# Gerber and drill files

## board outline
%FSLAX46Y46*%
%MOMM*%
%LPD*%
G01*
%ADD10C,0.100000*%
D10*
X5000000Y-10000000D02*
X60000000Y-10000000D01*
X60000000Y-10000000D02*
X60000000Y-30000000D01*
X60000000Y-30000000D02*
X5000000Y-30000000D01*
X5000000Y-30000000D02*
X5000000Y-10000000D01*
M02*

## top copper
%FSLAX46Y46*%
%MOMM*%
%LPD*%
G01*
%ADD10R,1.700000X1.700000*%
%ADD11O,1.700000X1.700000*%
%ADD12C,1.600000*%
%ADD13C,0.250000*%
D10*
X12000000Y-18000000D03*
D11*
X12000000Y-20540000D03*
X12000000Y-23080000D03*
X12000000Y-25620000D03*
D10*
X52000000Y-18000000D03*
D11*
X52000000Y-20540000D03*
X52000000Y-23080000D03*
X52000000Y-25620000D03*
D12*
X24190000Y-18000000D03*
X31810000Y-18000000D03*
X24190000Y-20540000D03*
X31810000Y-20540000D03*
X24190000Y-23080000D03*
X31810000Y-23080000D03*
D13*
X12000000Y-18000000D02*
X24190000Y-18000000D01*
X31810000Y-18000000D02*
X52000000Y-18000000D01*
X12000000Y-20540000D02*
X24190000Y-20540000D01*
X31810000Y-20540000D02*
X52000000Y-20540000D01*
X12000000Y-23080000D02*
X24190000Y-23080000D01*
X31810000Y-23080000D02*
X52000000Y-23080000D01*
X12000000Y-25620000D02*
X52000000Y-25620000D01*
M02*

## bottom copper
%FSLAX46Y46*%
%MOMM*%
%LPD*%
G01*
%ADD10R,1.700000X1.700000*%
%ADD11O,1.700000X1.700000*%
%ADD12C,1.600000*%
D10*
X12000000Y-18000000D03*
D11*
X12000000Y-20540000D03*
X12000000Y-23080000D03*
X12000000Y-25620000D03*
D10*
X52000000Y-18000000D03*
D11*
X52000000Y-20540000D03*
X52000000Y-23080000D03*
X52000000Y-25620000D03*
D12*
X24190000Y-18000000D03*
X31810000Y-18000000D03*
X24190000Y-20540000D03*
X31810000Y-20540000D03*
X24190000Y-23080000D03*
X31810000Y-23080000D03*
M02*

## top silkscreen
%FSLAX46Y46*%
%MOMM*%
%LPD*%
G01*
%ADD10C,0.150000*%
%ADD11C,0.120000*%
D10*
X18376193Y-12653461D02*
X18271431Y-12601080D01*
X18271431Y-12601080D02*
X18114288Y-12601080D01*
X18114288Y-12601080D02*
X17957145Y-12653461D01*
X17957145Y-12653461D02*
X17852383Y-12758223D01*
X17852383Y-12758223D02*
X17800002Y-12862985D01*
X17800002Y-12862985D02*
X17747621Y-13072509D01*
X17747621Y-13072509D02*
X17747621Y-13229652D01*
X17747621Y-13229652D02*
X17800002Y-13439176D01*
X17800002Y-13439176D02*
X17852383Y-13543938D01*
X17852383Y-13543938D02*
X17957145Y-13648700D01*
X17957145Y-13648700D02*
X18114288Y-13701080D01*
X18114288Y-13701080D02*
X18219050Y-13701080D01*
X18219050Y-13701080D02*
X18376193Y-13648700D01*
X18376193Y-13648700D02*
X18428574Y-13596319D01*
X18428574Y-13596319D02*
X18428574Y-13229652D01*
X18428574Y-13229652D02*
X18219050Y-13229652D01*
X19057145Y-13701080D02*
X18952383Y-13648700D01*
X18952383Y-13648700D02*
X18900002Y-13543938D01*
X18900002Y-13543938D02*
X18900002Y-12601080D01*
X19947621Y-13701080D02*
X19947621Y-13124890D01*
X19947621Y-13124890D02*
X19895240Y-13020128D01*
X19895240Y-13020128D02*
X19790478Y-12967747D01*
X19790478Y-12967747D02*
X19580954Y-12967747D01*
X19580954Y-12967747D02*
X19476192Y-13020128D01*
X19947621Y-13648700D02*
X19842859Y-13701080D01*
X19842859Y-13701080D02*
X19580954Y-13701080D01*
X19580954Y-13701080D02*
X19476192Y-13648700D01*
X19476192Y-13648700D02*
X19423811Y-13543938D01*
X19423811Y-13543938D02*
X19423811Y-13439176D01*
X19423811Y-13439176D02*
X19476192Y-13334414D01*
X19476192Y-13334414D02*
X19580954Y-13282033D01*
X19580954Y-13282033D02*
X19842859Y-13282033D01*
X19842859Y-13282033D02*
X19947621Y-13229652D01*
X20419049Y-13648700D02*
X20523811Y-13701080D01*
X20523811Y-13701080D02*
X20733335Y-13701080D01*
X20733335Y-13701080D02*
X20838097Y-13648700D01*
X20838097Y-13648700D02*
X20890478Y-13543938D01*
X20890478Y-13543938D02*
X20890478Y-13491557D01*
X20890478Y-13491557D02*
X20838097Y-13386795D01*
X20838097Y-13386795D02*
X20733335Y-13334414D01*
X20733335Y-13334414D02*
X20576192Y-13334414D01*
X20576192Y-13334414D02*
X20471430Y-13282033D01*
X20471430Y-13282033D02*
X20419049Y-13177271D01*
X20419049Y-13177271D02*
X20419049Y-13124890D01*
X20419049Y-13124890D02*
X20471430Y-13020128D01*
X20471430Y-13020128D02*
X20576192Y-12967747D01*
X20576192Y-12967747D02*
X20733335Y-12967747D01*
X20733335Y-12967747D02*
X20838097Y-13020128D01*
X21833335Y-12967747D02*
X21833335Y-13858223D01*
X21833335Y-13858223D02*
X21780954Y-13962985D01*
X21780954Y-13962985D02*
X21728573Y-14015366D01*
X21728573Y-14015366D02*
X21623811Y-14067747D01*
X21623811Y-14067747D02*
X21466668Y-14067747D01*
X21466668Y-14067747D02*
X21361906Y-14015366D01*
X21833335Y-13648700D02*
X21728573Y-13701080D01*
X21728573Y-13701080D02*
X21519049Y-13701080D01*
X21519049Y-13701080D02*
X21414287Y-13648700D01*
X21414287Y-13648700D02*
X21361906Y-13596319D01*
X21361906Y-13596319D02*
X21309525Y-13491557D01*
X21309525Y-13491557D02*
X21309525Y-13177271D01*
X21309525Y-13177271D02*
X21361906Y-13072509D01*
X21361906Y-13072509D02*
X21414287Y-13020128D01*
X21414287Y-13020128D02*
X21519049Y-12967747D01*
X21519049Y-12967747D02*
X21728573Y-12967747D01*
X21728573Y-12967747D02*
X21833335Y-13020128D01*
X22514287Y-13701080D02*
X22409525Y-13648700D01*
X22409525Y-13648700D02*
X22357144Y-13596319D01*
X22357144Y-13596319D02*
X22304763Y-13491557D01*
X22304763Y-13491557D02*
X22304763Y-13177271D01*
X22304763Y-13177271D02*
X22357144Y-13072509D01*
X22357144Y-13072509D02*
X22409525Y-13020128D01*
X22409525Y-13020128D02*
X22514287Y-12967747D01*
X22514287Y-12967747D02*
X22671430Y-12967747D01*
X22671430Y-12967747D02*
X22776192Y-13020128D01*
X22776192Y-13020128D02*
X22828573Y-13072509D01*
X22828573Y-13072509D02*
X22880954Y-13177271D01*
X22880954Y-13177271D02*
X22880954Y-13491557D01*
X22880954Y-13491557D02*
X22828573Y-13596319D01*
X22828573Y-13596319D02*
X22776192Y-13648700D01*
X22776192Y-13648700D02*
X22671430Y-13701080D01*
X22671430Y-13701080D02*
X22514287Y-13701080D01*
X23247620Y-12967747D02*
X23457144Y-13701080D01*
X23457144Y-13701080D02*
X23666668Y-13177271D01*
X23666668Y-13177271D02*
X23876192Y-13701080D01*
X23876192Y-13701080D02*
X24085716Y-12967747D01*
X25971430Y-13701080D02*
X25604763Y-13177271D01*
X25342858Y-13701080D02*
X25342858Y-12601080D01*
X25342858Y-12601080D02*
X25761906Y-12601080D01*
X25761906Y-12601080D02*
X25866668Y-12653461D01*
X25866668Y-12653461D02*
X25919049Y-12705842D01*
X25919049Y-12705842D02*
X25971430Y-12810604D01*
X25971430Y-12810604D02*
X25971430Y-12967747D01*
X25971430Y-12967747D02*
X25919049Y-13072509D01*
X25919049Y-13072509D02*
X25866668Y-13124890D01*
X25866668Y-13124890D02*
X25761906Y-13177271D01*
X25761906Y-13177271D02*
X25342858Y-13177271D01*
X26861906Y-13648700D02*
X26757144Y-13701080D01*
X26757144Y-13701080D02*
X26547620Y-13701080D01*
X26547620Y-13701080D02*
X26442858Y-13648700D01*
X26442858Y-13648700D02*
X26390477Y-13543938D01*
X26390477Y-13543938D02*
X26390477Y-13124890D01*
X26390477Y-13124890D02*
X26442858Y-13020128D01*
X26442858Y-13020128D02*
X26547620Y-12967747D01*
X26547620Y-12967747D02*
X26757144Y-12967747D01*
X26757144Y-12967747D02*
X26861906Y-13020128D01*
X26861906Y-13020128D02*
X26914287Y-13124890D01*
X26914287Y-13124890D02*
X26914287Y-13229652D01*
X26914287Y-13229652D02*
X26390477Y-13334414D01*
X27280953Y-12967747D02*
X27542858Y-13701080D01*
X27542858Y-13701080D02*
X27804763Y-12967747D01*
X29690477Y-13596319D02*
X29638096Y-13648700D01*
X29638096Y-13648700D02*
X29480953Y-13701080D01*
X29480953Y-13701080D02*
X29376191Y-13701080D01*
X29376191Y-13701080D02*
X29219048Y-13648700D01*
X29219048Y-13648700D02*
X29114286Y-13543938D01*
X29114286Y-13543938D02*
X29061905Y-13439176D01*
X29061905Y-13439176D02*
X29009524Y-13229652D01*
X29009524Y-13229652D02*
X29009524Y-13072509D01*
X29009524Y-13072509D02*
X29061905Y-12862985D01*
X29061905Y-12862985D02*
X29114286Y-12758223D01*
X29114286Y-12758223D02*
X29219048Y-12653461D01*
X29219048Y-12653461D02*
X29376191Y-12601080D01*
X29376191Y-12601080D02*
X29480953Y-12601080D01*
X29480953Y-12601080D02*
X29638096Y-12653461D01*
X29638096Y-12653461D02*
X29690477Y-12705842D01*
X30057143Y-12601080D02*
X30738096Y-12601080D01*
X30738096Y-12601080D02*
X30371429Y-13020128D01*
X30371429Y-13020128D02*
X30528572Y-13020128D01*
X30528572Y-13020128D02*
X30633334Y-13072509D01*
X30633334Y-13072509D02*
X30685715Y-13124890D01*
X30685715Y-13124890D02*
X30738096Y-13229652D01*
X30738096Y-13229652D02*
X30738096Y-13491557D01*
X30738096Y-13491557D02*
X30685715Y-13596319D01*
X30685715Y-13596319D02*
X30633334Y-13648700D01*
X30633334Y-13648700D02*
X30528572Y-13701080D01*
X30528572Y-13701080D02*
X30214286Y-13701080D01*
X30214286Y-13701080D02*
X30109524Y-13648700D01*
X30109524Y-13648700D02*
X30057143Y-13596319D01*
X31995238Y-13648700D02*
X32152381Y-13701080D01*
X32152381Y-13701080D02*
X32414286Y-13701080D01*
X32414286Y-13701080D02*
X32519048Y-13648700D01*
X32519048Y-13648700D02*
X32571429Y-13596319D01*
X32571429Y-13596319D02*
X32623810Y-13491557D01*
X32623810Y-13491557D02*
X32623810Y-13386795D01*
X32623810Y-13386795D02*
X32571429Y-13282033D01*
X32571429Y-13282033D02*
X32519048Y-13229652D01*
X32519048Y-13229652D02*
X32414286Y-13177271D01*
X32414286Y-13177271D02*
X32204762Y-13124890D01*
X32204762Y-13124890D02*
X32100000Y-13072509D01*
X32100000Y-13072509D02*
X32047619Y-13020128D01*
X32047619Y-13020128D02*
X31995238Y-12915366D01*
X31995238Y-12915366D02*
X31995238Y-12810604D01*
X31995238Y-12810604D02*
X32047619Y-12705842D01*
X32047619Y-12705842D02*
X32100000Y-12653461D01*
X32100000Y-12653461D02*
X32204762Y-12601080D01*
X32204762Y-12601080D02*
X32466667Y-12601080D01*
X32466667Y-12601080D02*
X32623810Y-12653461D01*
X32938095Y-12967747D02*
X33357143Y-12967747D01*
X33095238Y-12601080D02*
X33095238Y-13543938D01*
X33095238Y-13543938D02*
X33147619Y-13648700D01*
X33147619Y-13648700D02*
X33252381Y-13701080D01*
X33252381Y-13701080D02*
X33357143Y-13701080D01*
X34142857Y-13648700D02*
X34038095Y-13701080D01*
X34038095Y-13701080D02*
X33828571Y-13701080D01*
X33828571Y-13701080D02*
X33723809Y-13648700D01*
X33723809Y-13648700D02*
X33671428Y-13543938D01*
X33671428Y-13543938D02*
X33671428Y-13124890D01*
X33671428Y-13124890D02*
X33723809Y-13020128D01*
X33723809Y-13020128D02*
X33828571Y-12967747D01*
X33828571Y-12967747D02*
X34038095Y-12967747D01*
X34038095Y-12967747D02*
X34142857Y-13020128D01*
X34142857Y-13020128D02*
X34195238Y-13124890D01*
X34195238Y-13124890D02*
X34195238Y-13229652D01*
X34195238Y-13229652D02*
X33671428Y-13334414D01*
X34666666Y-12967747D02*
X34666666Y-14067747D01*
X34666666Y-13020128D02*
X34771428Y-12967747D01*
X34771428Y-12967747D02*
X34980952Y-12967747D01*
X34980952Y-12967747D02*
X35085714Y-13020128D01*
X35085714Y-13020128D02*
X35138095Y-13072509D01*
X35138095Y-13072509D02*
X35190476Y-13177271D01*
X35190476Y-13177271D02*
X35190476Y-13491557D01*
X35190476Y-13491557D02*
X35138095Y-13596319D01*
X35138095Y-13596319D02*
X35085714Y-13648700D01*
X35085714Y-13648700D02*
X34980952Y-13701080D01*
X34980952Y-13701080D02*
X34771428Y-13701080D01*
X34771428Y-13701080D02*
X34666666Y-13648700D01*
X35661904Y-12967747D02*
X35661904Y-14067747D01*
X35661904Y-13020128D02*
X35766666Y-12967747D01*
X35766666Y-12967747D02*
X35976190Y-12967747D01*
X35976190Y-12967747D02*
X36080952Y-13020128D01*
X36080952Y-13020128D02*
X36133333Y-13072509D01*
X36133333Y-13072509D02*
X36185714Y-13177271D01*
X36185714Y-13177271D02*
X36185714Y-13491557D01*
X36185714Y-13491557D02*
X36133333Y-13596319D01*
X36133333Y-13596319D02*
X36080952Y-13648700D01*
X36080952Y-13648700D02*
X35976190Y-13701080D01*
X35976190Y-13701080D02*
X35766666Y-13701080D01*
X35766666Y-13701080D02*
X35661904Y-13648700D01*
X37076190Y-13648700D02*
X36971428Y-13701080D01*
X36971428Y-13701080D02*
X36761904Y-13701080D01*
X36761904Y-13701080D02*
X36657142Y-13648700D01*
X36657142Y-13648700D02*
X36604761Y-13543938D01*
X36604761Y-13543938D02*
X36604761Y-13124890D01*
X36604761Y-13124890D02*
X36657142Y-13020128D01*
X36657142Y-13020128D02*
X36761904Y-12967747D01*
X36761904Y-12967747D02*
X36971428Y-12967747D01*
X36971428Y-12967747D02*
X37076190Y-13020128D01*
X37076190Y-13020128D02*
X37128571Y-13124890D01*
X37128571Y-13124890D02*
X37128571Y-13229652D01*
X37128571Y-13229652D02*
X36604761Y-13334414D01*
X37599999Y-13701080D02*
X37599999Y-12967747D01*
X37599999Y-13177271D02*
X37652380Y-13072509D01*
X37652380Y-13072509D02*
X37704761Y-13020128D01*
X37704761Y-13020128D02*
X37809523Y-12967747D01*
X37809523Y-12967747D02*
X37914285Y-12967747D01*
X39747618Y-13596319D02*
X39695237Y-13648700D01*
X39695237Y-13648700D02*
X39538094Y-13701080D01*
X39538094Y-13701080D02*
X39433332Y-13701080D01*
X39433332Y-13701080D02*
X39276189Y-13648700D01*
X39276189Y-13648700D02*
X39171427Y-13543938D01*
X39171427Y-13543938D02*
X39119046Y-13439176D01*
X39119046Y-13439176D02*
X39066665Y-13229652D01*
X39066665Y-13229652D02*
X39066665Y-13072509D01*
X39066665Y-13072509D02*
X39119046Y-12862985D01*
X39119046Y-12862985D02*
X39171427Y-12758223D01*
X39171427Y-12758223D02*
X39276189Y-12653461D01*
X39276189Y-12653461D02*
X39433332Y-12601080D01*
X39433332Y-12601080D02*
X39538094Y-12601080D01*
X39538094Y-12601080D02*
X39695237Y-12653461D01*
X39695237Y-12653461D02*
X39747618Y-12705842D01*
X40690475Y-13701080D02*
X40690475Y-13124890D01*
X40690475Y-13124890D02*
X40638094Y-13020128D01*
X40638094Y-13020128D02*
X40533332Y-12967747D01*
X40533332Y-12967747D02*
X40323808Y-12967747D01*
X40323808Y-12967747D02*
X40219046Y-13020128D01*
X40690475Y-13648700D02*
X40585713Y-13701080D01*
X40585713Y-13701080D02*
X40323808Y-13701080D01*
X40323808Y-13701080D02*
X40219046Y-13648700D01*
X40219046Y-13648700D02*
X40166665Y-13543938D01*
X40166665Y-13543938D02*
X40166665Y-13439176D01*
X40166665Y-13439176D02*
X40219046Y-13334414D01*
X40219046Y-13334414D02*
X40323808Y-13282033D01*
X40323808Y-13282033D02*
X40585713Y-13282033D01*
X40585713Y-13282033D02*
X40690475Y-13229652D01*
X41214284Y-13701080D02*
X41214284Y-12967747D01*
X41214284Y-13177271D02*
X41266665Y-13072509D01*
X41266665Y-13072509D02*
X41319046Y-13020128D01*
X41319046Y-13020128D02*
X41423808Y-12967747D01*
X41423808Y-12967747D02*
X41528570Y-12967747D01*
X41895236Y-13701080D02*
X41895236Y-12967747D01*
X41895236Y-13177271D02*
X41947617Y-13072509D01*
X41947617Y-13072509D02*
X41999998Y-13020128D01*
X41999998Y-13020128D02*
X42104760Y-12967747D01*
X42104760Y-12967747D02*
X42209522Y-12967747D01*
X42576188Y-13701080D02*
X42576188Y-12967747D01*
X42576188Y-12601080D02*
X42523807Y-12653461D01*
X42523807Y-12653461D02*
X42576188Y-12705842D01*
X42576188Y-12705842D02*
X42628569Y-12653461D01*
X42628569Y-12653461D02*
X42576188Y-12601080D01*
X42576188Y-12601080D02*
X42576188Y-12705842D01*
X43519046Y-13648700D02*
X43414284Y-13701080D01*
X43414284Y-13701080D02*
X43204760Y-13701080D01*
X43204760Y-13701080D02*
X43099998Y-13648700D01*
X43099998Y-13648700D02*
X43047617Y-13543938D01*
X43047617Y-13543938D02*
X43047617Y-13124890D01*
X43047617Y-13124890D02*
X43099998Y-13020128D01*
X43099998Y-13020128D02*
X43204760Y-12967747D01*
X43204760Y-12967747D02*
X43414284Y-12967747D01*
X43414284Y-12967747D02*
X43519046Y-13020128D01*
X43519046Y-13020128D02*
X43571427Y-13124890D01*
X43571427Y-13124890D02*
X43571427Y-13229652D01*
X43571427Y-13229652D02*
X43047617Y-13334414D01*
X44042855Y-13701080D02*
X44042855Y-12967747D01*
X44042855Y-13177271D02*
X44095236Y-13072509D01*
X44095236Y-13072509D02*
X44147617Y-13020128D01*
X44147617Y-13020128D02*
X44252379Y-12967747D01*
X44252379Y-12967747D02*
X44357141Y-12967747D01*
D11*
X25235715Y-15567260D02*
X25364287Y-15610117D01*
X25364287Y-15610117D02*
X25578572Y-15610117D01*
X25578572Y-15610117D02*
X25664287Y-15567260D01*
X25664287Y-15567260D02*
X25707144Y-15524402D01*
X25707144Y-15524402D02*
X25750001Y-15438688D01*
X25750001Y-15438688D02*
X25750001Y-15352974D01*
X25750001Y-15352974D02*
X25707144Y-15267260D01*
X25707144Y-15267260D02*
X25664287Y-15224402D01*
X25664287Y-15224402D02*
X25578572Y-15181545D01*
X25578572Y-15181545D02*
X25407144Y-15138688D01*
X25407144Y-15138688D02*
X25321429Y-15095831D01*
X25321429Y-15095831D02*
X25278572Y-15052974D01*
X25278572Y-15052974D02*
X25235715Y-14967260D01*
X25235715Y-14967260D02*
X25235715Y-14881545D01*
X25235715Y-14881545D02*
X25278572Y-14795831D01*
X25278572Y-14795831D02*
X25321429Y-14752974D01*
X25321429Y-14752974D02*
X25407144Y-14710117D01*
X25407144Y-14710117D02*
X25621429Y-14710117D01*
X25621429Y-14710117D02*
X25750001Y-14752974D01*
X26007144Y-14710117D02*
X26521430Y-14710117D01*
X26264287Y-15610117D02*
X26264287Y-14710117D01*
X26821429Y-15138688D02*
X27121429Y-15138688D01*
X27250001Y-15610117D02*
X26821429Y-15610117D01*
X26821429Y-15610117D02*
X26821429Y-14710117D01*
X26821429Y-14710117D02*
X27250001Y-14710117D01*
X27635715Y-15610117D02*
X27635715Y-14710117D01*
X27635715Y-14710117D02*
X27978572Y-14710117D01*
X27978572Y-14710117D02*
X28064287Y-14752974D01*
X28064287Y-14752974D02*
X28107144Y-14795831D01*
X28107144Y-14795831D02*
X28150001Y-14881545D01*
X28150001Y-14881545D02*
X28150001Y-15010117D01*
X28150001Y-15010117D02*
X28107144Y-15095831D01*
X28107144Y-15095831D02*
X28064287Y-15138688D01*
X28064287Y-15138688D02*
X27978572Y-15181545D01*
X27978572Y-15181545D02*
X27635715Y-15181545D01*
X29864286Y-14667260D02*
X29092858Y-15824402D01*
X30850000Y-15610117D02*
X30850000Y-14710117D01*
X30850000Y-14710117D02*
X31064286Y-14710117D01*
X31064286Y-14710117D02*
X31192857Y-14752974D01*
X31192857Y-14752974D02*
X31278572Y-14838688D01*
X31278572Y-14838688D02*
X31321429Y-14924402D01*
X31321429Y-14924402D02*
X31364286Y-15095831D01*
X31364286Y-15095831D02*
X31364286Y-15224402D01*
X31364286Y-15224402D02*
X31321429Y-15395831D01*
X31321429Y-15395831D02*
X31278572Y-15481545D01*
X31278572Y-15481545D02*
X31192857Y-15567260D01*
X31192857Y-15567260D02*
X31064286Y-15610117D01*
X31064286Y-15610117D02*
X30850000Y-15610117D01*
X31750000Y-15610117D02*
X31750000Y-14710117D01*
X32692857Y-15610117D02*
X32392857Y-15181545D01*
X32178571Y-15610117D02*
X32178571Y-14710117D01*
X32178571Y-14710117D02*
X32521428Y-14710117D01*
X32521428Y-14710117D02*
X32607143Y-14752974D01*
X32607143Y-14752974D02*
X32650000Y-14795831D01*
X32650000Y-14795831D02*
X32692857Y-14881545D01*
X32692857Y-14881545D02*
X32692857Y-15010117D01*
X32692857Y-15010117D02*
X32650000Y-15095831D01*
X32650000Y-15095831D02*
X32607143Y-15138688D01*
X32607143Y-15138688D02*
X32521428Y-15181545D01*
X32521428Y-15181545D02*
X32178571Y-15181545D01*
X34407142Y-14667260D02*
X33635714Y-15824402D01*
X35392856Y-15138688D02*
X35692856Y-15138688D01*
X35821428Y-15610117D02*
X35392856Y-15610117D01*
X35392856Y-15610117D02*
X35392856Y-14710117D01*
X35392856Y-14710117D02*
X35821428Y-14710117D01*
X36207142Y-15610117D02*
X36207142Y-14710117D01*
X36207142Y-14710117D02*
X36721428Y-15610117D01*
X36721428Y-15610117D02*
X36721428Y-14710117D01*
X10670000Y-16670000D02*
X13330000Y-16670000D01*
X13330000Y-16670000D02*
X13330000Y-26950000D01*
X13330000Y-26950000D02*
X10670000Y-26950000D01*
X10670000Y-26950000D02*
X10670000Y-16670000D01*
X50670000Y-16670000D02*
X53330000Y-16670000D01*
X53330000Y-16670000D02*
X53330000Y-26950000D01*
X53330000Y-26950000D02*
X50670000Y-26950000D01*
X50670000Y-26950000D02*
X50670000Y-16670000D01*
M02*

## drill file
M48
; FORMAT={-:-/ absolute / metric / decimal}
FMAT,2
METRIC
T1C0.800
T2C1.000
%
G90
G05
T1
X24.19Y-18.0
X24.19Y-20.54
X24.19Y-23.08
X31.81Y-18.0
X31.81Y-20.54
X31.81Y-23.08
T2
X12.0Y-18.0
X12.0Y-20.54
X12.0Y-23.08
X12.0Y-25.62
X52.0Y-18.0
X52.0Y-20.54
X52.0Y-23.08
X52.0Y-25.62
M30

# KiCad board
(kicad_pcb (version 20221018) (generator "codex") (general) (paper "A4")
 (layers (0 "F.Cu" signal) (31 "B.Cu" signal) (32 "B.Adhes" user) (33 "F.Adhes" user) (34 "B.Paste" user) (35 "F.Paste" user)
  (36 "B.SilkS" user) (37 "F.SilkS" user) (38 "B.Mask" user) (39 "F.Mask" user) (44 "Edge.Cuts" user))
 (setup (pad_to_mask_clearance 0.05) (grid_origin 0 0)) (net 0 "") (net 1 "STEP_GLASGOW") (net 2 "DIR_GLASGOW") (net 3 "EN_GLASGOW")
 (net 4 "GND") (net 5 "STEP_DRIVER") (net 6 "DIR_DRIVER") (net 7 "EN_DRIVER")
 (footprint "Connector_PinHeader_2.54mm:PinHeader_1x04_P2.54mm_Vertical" (layer "F.Cu") (at 12 18)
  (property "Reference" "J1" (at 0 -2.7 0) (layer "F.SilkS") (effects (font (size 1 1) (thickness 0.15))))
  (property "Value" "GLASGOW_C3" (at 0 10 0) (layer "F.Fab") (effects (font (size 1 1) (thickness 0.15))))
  (fp_line (start -1.33 -1.33) (end 1.33 -1.33) (layer "F.SilkS") (width 0.12))
  (fp_line (start 1.33 -1.33) (end 1.33 8.95) (layer "F.SilkS") (width 0.12))
  (fp_line (start 1.33 8.95) (end -1.33 8.95) (layer "F.SilkS") (width 0.12))
  (fp_line (start -1.33 8.95) (end -1.33 -1.33) (layer "F.SilkS") (width 0.12))
  (pad "1" thru_hole rect (at 0 0) (size 1.7 1.7) (drill 1.0) (layers "*.Cu" "*.Mask") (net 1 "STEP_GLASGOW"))
  (pad "2" thru_hole oval (at 0 2.54) (size 1.7 1.7) (drill 1.0) (layers "*.Cu" "*.Mask") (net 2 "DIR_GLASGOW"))
  (pad "3" thru_hole oval (at 0 5.08) (size 1.7 1.7) (drill 1.0) (layers "*.Cu" "*.Mask") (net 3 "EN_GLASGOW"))
  (pad "4" thru_hole oval (at 0 7.62) (size 1.7 1.7) (drill 1.0) (layers "*.Cu" "*.Mask") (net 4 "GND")))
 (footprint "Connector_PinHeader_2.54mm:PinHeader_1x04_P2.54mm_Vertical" (layer "F.Cu") (at 52 18)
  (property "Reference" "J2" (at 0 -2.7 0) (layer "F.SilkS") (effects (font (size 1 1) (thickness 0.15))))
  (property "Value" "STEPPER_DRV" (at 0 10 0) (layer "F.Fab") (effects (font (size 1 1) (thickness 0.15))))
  (fp_line (start -1.33 -1.33) (end 1.33 -1.33) (layer "F.SilkS") (width 0.12))
  (fp_line (start 1.33 -1.33) (end 1.33 8.95) (layer "F.SilkS") (width 0.12))
  (fp_line (start 1.33 8.95) (end -1.33 8.95) (layer "F.SilkS") (width 0.12))
  (fp_line (start -1.33 8.95) (end -1.33 -1.33) (layer "F.SilkS") (width 0.12))
  (pad "1" thru_hole rect (at 0 0) (size 1.7 1.7) (drill 1.0) (layers "*.Cu" "*.Mask") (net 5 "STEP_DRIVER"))
  (pad "2" thru_hole oval (at 0 2.54) (size 1.7 1.7) (drill 1.0) (layers "*.Cu" "*.Mask") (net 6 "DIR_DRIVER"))
  (pad "3" thru_hole oval (at 0 5.08) (size 1.7 1.7) (drill 1.0) (layers "*.Cu" "*.Mask") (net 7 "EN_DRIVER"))
  (pad "4" thru_hole oval (at 0 7.62) (size 1.7 1.7) (drill 1.0) (layers "*.Cu" "*.Mask") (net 4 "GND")))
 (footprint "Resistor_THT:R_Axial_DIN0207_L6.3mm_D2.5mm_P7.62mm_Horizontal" (layer "F.Cu") (at 28 18)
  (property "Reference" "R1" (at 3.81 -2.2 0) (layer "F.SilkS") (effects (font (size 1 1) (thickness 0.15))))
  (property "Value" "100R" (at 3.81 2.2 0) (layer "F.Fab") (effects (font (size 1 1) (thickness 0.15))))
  (pad "1" thru_hole circle (at -3.81 0) (size 1.6 1.6) (drill 0.8) (layers "*.Cu" "*.Mask") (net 1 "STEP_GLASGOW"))
  (pad "2" thru_hole circle (at 3.81 0) (size 1.6 1.6) (drill 0.8) (layers "*.Cu" "*.Mask") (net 5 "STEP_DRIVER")))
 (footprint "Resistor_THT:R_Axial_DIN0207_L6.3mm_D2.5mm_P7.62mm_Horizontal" (layer "F.Cu") (at 28 20.54)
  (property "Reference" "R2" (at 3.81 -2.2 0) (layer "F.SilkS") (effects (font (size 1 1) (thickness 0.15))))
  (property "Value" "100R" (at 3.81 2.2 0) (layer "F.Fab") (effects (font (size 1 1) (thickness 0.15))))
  (pad "1" thru_hole circle (at -3.81 0) (size 1.6 1.6) (drill 0.8) (layers "*.Cu" "*.Mask") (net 2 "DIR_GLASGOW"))
  (pad "2" thru_hole circle (at 3.81 0) (size 1.6 1.6) (drill 0.8) (layers "*.Cu" "*.Mask") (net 6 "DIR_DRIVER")))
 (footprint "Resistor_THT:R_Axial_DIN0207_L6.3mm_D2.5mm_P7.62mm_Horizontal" (layer "F.Cu") (at 28 23.08)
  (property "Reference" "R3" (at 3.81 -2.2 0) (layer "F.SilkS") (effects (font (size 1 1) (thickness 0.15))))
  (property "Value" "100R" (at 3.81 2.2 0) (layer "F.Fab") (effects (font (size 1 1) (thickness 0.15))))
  (pad "1" thru_hole circle (at -3.81 0) (size 1.6 1.6) (drill 0.8) (layers "*.Cu" "*.Mask") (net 3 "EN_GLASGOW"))
  (pad "2" thru_hole circle (at 3.81 0) (size 1.6 1.6) (drill 0.8) (layers "*.Cu" "*.Mask") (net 7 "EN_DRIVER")))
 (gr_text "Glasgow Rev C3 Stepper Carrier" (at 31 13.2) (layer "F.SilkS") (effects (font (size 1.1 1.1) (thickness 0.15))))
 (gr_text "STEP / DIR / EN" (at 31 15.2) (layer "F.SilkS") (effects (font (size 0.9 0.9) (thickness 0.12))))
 (gr_line (start 5 10) (end 60 10) (layer "Edge.Cuts") (width 0.1))
 (gr_line (start 60 10) (end 60 30) (layer "Edge.Cuts") (width 0.1))
 (gr_line (start 60 30) (end 5 30) (layer "Edge.Cuts") (width 0.1))
 (gr_line (start 5 30) (end 5 10) (layer "Edge.Cuts") (width 0.1))
 (segment (start 12 18) (end 24.19 18) (width 0.25) (layer "F.Cu") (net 1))
 (segment (start 31.81 18) (end 52 18) (width 0.25) (layer "F.Cu") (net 5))
 (segment (start 12 20.54) (end 24.19 20.54) (width 0.25) (layer "F.Cu") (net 2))
 (segment (start 31.81 20.54) (end 52 20.54) (width 0.25) (layer "F.Cu") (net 6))
 (segment (start 12 23.08) (end 24.19 23.08) (width 0.25) (layer "F.Cu") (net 3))
 (segment (start 31.81 23.08) (end 52 23.08) (width 0.25) (layer "F.Cu") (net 7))
 (segment (start 12 25.62) (end 52 25.62) (width 0.25) (layer "F.Cu") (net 4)))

